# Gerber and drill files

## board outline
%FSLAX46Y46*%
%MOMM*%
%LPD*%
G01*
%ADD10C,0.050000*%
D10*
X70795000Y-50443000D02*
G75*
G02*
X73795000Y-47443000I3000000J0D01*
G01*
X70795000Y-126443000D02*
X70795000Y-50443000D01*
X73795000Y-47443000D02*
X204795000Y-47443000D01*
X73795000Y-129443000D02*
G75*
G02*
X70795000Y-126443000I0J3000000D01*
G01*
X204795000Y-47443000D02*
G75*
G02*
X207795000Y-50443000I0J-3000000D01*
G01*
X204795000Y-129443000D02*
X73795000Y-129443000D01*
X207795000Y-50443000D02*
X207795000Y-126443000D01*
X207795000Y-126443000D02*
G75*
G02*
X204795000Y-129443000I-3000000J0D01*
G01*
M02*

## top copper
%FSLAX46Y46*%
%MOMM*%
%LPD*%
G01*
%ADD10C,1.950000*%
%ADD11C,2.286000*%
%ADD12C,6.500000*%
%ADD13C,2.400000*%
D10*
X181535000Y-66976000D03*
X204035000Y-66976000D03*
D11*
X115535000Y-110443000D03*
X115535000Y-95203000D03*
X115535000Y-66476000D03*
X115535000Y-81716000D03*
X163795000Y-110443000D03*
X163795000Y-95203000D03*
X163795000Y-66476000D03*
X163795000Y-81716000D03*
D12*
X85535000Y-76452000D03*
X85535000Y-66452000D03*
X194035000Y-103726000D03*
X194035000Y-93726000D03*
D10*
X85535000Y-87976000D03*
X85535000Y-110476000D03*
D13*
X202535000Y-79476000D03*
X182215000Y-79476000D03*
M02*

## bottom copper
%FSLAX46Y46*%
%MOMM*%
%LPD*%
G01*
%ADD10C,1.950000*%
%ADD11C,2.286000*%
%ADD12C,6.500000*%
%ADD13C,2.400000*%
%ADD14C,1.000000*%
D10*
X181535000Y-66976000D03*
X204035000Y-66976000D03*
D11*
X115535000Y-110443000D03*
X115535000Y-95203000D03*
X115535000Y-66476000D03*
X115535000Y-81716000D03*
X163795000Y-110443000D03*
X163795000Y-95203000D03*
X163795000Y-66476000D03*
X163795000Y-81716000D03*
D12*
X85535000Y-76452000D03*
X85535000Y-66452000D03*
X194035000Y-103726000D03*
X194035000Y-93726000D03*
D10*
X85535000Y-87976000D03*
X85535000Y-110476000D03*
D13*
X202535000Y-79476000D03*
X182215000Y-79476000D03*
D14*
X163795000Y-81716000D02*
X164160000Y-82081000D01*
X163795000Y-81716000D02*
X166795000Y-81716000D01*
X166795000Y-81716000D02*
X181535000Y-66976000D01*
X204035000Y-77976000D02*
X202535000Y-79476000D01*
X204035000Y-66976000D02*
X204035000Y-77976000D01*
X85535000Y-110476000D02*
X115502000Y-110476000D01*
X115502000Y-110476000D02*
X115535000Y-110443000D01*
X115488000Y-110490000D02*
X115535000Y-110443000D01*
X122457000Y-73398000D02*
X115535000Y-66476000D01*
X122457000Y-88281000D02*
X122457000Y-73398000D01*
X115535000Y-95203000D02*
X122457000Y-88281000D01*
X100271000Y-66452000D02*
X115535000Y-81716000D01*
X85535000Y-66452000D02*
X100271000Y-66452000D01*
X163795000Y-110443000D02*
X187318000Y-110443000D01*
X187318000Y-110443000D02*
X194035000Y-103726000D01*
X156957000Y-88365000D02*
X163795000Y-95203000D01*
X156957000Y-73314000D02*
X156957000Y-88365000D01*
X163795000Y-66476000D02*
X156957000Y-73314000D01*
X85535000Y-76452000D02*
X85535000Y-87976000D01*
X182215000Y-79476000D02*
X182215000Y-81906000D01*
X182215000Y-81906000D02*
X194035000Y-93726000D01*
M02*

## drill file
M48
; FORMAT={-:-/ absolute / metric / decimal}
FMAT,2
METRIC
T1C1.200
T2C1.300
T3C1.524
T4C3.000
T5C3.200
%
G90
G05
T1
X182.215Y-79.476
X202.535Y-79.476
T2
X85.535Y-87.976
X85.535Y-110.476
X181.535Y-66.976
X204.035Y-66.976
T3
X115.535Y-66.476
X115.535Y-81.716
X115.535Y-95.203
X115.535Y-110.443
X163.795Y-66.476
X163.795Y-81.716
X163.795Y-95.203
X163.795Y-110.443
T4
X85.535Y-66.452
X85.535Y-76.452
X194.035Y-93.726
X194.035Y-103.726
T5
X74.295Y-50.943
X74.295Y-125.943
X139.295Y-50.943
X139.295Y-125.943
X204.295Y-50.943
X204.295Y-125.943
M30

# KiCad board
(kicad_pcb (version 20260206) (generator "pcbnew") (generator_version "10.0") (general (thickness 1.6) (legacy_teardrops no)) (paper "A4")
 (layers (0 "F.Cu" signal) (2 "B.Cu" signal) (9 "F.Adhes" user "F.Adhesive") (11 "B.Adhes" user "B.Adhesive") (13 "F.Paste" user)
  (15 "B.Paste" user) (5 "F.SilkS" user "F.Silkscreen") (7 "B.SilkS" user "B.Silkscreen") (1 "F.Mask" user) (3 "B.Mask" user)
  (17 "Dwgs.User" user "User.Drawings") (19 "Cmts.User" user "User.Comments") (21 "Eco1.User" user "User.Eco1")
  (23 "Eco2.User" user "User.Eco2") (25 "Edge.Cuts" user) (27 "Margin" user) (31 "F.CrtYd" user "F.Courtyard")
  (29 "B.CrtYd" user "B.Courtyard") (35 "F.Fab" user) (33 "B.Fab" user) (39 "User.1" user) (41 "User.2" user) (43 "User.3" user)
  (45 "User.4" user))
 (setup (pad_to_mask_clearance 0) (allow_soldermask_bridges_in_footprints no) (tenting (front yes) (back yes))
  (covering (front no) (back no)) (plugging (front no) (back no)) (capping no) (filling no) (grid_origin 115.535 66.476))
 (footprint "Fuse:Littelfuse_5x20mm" (layer "F.Cu") (at 192.785 66.976)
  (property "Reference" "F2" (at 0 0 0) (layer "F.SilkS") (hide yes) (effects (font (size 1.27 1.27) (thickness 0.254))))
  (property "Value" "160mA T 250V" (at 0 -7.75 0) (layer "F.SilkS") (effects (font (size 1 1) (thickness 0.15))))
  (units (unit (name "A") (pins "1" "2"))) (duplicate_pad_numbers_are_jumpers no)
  (pad "1" thru_hole circle (at -11.25 0) (size 1.95 1.95) (drill 1.3) (layers "*.Cu" "*.Mask") (remove_unused_layers no) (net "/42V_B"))
  (pad "2" thru_hole circle (at 11.25 0) (size 1.95 1.95) (drill 1.3) (layers "*.Cu" "*.Mask") (remove_unused_layers no)
   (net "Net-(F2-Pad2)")))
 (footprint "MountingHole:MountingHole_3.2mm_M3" (layer "F.Cu") (at 139.295 125.943)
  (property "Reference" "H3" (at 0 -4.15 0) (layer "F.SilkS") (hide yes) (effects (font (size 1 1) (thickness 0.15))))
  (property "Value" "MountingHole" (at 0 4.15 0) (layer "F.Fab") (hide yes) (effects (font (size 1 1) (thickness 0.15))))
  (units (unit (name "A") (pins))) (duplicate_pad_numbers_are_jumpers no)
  (pad "" np_thru_hole circle (at 0 0) (size 3.2 3.2) (drill 3.2) (layers "*.Cu" "*.Mask")))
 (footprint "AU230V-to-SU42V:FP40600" (layer "F.Cu") (at 115.535 110.443 -90)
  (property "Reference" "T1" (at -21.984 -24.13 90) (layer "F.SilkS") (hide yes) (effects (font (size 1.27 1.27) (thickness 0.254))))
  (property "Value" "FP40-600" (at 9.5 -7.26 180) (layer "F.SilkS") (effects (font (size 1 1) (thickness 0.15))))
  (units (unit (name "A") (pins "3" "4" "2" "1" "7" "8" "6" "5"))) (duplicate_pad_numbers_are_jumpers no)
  (pad "1" thru_hole circle (at 0 0 270) (size 2.286 2.286) (drill 1.524) (layers "*.Cu" "*.Mask") (remove_unused_layers no)
   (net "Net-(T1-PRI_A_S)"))
  (pad "2" thru_hole circle (at -15.24 0 270) (size 2.286 2.286) (drill 1.524) (layers "*.Cu" "*.Mask") (remove_unused_layers no)
   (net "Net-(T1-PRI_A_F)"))
  (pad "3" thru_hole circle (at -43.967 0 270) (size 2.286 2.286) (drill 1.524) (layers "*.Cu" "*.Mask") (remove_unused_layers no)
   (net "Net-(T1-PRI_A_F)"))
  (pad "4" thru_hole circle (at -28.727 0 270) (size 2.286 2.286) (drill 1.524) (layers "*.Cu" "*.Mask") (remove_unused_layers no)
   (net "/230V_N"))
  (pad "5" thru_hole circle (at 0 -48.26 270) (size 2.286 2.286) (drill 1.524) (layers "*.Cu" "*.Mask") (remove_unused_layers no)
   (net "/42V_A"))
  (pad "6" thru_hole circle (at -15.24 -48.26 270) (size 2.286 2.286) (drill 1.524) (layers "*.Cu" "*.Mask") (remove_unused_layers no)
   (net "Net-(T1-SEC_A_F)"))
  (pad "7" thru_hole circle (at -43.967 -48.26 270) (size 2.286 2.286) (drill 1.524) (layers "*.Cu" "*.Mask") (remove_unused_layers no)
   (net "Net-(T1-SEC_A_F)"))
  (pad "8" thru_hole circle (at -28.727 -48.26 270) (size 2.286 2.286) (drill 1.524) (layers "*.Cu" "*.Mask") (remove_unused_layers no)
   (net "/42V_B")))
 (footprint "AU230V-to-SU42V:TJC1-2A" (layer "F.Cu") (at 85.535 76.452 90)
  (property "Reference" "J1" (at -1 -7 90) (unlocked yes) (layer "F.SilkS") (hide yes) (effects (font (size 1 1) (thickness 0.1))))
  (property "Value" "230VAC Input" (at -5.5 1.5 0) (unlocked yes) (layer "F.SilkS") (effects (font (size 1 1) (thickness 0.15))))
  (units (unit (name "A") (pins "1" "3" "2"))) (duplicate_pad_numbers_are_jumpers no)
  (pad "1" thru_hole circle (at 0 0 90) (size 6.5 6.5) (drill 3) (layers "*.Cu" "*.Mask") (remove_unused_layers no) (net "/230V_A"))
  (pad "2" thru_hole circle (at 10 0 90) (size 6.5 6.5) (drill 3) (layers "*.Cu" "*.Mask") (remove_unused_layers no) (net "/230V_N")))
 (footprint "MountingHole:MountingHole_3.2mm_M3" (layer "F.Cu") (at 74.295 50.943)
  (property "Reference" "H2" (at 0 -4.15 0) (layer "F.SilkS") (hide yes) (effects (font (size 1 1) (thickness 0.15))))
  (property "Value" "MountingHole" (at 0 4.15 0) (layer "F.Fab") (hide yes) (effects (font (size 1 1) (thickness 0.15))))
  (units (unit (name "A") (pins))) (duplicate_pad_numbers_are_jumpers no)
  (pad "" np_thru_hole circle (at 0 0) (size 3.2 3.2) (drill 3.2) (layers "*.Cu" "*.Mask")))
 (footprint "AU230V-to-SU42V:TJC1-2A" (layer "F.Cu") (at 194.035 103.726 90)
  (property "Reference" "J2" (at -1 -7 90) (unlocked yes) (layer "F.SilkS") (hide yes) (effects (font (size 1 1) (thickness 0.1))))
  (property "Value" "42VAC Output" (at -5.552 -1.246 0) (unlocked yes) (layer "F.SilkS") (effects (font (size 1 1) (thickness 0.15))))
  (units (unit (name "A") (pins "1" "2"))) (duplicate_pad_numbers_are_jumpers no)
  (pad "1" thru_hole circle (at 0 0 90) (size 6.5 6.5) (drill 3) (layers "*.Cu" "*.Mask") (remove_unused_layers no) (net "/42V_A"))
  (pad "2" thru_hole circle (at 10 0 90) (size 6.5 6.5) (drill 3) (layers "*.Cu" "*.Mask") (remove_unused_layers no) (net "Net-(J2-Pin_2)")))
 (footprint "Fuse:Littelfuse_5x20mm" (layer "F.Cu") (at 85.535 99.226 -90)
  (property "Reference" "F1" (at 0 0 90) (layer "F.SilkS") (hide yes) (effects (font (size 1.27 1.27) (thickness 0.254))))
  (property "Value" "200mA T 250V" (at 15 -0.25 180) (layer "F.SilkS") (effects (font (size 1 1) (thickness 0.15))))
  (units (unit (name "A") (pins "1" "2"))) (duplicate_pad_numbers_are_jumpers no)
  (pad "1" thru_hole circle (at -11.25 0 270) (size 1.95 1.95) (drill 1.3) (layers "*.Cu" "*.Mask") (remove_unused_layers no)
   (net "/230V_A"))
  (pad "2" thru_hole circle (at 11.25 0 270) (size 1.95 1.95) (drill 1.3) (layers "*.Cu" "*.Mask") (remove_unused_layers no)
   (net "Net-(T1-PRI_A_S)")))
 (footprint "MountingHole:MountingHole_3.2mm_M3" (layer "F.Cu") (at 204.295 50.943)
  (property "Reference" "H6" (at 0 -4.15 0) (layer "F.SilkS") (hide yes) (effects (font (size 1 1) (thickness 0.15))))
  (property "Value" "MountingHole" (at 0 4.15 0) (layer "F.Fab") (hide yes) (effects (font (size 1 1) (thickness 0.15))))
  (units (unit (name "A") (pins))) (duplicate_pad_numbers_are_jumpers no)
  (pad "" np_thru_hole circle (at 0 0) (size 3.2 3.2) (drill 3.2) (layers "*.Cu" "*.Mask")))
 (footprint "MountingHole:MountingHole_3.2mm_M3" (layer "F.Cu") (at 74.295 125.943)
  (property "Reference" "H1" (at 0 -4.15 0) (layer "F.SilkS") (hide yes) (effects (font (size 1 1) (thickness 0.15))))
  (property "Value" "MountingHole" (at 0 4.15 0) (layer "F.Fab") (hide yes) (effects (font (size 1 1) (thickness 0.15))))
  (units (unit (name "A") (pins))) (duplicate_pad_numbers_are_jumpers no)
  (pad "" np_thru_hole circle (at 0 0) (size 3.2 3.2) (drill 3.2) (layers "*.Cu" "*.Mask")))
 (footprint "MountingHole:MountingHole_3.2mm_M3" (layer "F.Cu") (at 139.295 50.943)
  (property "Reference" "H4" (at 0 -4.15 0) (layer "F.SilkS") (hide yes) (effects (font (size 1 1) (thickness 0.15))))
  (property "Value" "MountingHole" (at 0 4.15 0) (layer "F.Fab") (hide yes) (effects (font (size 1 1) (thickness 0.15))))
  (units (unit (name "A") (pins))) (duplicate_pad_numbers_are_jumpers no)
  (pad "" np_thru_hole circle (at 0 0) (size 3.2 3.2) (drill 3.2) (layers "*.Cu" "*.Mask")))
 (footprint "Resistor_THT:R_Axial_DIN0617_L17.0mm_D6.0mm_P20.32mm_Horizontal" (layer "F.Cu") (at 202.535 79.476 180)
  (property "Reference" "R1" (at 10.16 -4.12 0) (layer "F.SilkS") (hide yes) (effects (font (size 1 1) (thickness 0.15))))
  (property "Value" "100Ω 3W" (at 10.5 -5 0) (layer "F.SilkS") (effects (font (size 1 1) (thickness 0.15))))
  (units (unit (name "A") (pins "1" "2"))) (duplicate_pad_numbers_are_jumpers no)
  (pad "1" thru_hole circle (at 0 0 180) (size 2.4 2.4) (drill 1.2) (layers "*.Cu" "*.Mask") (remove_unused_layers no) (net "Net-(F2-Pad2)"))
  (pad "2" thru_hole circle (at 20.32 0 180) (size 2.4 2.4) (drill 1.2) (layers "*.Cu" "*.Mask") (remove_unused_layers no)
   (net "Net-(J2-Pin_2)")))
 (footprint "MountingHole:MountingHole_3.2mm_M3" (layer "F.Cu") (at 204.295 125.943)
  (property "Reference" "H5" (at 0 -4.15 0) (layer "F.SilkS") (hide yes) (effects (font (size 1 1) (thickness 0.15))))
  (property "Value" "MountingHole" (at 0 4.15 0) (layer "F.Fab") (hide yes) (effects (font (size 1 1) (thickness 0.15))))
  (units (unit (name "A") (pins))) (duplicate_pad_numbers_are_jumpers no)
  (pad "" np_thru_hole circle (at 0 0) (size 3.2 3.2) (drill 3.2) (layers "*.Cu" "*.Mask")))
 (gr_arc (start 70.795 50.443) (mid 71.67368 48.32168) (end 73.795 47.443) (stroke (width 0.05) (type default)) (layer "Edge.Cuts"))
 (gr_line (start 70.795 126.443) (end 70.795 50.443) (stroke (width 0.05) (type default)) (layer "Edge.Cuts"))
 (gr_line (start 73.795 47.443) (end 204.795 47.443) (stroke (width 0.05) (type default)) (layer "Edge.Cuts"))
 (gr_arc (start 73.795 129.443) (mid 71.67368 128.56432) (end 70.795 126.443) (stroke (width 0.05) (type default)) (layer "Edge.Cuts"))
 (gr_arc (start 204.795 47.443) (mid 206.91632 48.32168) (end 207.795 50.443) (stroke (width 0.05) (type default)) (layer "Edge.Cuts"))
 (gr_line (start 204.795 129.443) (end 73.795 129.443) (stroke (width 0.05) (type default)) (layer "Edge.Cuts"))
 (gr_line (start 207.795 50.443) (end 207.795 126.443) (stroke (width 0.05) (type default)) (layer "Edge.Cuts"))
 (gr_arc (start 207.795 126.443) (mid 206.91632 128.56432) (end 204.795 129.443) (stroke (width 0.05) (type default)) (layer "Edge.Cuts"))
 (segment (start 163.795 81.716) (end 164.16 82.081) (width 1) (layer "B.Cu") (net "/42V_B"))
 (segment (start 163.795 81.716) (end 166.795 81.716) (width 1) (layer "B.Cu") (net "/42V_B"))
 (segment (start 166.795 81.716) (end 181.535 66.976) (width 1) (layer "B.Cu") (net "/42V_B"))
 (segment (start 204.035 77.976) (end 202.535 79.476) (width 1) (layer "B.Cu") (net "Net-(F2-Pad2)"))
 (segment (start 204.035 66.976) (end 204.035 77.976) (width 1) (layer "B.Cu") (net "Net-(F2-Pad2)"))
 (segment (start 85.535 110.476) (end 115.502 110.476) (width 1) (layer "B.Cu") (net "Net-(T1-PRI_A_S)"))
 (segment (start 115.502 110.476) (end 115.535 110.443) (width 1) (layer "B.Cu") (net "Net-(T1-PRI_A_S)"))
 (segment (start 115.488 110.49) (end 115.535 110.443) (width 1) (layer "B.Cu") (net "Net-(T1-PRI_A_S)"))
 (segment (start 122.457 73.398) (end 115.535 66.476) (width 1) (layer "B.Cu") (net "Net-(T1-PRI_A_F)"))
 (segment (start 122.457 88.281) (end 122.457 73.398) (width 1) (layer "B.Cu") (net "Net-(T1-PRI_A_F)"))
 (segment (start 115.535 95.203) (end 122.457 88.281) (width 1) (layer "B.Cu") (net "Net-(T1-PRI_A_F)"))
 (segment (start 100.271 66.452) (end 115.535 81.716) (width 1) (layer "B.Cu") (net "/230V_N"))
 (segment (start 85.535 66.452) (end 100.271 66.452) (width 1) (layer "B.Cu") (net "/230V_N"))
 (segment (start 163.795 110.443) (end 187.318 110.443) (width 1) (layer "B.Cu") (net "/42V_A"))
 (segment (start 187.318 110.443) (end 194.035 103.726) (width 1) (layer "B.Cu") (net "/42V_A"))
 (segment (start 156.957 88.365) (end 163.795 95.203) (width 1) (layer "B.Cu") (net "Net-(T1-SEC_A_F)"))
 (segment (start 156.957 73.314) (end 156.957 88.365) (width 1) (layer "B.Cu") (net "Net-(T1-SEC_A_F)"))
 (segment (start 163.795 66.476) (end 156.957 73.314) (width 1) (layer "B.Cu") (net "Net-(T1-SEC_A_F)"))
 (segment (start 85.535 76.452) (end 85.535 87.976) (width 1) (layer "B.Cu") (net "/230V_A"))
 (segment (start 182.215 79.476) (end 182.215 81.906) (width 1) (layer "B.Cu") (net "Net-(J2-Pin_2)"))
 (segment (start 182.215 81.906) (end 194.035 93.726) (width 1) (layer "B.Cu") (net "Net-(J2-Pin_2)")))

